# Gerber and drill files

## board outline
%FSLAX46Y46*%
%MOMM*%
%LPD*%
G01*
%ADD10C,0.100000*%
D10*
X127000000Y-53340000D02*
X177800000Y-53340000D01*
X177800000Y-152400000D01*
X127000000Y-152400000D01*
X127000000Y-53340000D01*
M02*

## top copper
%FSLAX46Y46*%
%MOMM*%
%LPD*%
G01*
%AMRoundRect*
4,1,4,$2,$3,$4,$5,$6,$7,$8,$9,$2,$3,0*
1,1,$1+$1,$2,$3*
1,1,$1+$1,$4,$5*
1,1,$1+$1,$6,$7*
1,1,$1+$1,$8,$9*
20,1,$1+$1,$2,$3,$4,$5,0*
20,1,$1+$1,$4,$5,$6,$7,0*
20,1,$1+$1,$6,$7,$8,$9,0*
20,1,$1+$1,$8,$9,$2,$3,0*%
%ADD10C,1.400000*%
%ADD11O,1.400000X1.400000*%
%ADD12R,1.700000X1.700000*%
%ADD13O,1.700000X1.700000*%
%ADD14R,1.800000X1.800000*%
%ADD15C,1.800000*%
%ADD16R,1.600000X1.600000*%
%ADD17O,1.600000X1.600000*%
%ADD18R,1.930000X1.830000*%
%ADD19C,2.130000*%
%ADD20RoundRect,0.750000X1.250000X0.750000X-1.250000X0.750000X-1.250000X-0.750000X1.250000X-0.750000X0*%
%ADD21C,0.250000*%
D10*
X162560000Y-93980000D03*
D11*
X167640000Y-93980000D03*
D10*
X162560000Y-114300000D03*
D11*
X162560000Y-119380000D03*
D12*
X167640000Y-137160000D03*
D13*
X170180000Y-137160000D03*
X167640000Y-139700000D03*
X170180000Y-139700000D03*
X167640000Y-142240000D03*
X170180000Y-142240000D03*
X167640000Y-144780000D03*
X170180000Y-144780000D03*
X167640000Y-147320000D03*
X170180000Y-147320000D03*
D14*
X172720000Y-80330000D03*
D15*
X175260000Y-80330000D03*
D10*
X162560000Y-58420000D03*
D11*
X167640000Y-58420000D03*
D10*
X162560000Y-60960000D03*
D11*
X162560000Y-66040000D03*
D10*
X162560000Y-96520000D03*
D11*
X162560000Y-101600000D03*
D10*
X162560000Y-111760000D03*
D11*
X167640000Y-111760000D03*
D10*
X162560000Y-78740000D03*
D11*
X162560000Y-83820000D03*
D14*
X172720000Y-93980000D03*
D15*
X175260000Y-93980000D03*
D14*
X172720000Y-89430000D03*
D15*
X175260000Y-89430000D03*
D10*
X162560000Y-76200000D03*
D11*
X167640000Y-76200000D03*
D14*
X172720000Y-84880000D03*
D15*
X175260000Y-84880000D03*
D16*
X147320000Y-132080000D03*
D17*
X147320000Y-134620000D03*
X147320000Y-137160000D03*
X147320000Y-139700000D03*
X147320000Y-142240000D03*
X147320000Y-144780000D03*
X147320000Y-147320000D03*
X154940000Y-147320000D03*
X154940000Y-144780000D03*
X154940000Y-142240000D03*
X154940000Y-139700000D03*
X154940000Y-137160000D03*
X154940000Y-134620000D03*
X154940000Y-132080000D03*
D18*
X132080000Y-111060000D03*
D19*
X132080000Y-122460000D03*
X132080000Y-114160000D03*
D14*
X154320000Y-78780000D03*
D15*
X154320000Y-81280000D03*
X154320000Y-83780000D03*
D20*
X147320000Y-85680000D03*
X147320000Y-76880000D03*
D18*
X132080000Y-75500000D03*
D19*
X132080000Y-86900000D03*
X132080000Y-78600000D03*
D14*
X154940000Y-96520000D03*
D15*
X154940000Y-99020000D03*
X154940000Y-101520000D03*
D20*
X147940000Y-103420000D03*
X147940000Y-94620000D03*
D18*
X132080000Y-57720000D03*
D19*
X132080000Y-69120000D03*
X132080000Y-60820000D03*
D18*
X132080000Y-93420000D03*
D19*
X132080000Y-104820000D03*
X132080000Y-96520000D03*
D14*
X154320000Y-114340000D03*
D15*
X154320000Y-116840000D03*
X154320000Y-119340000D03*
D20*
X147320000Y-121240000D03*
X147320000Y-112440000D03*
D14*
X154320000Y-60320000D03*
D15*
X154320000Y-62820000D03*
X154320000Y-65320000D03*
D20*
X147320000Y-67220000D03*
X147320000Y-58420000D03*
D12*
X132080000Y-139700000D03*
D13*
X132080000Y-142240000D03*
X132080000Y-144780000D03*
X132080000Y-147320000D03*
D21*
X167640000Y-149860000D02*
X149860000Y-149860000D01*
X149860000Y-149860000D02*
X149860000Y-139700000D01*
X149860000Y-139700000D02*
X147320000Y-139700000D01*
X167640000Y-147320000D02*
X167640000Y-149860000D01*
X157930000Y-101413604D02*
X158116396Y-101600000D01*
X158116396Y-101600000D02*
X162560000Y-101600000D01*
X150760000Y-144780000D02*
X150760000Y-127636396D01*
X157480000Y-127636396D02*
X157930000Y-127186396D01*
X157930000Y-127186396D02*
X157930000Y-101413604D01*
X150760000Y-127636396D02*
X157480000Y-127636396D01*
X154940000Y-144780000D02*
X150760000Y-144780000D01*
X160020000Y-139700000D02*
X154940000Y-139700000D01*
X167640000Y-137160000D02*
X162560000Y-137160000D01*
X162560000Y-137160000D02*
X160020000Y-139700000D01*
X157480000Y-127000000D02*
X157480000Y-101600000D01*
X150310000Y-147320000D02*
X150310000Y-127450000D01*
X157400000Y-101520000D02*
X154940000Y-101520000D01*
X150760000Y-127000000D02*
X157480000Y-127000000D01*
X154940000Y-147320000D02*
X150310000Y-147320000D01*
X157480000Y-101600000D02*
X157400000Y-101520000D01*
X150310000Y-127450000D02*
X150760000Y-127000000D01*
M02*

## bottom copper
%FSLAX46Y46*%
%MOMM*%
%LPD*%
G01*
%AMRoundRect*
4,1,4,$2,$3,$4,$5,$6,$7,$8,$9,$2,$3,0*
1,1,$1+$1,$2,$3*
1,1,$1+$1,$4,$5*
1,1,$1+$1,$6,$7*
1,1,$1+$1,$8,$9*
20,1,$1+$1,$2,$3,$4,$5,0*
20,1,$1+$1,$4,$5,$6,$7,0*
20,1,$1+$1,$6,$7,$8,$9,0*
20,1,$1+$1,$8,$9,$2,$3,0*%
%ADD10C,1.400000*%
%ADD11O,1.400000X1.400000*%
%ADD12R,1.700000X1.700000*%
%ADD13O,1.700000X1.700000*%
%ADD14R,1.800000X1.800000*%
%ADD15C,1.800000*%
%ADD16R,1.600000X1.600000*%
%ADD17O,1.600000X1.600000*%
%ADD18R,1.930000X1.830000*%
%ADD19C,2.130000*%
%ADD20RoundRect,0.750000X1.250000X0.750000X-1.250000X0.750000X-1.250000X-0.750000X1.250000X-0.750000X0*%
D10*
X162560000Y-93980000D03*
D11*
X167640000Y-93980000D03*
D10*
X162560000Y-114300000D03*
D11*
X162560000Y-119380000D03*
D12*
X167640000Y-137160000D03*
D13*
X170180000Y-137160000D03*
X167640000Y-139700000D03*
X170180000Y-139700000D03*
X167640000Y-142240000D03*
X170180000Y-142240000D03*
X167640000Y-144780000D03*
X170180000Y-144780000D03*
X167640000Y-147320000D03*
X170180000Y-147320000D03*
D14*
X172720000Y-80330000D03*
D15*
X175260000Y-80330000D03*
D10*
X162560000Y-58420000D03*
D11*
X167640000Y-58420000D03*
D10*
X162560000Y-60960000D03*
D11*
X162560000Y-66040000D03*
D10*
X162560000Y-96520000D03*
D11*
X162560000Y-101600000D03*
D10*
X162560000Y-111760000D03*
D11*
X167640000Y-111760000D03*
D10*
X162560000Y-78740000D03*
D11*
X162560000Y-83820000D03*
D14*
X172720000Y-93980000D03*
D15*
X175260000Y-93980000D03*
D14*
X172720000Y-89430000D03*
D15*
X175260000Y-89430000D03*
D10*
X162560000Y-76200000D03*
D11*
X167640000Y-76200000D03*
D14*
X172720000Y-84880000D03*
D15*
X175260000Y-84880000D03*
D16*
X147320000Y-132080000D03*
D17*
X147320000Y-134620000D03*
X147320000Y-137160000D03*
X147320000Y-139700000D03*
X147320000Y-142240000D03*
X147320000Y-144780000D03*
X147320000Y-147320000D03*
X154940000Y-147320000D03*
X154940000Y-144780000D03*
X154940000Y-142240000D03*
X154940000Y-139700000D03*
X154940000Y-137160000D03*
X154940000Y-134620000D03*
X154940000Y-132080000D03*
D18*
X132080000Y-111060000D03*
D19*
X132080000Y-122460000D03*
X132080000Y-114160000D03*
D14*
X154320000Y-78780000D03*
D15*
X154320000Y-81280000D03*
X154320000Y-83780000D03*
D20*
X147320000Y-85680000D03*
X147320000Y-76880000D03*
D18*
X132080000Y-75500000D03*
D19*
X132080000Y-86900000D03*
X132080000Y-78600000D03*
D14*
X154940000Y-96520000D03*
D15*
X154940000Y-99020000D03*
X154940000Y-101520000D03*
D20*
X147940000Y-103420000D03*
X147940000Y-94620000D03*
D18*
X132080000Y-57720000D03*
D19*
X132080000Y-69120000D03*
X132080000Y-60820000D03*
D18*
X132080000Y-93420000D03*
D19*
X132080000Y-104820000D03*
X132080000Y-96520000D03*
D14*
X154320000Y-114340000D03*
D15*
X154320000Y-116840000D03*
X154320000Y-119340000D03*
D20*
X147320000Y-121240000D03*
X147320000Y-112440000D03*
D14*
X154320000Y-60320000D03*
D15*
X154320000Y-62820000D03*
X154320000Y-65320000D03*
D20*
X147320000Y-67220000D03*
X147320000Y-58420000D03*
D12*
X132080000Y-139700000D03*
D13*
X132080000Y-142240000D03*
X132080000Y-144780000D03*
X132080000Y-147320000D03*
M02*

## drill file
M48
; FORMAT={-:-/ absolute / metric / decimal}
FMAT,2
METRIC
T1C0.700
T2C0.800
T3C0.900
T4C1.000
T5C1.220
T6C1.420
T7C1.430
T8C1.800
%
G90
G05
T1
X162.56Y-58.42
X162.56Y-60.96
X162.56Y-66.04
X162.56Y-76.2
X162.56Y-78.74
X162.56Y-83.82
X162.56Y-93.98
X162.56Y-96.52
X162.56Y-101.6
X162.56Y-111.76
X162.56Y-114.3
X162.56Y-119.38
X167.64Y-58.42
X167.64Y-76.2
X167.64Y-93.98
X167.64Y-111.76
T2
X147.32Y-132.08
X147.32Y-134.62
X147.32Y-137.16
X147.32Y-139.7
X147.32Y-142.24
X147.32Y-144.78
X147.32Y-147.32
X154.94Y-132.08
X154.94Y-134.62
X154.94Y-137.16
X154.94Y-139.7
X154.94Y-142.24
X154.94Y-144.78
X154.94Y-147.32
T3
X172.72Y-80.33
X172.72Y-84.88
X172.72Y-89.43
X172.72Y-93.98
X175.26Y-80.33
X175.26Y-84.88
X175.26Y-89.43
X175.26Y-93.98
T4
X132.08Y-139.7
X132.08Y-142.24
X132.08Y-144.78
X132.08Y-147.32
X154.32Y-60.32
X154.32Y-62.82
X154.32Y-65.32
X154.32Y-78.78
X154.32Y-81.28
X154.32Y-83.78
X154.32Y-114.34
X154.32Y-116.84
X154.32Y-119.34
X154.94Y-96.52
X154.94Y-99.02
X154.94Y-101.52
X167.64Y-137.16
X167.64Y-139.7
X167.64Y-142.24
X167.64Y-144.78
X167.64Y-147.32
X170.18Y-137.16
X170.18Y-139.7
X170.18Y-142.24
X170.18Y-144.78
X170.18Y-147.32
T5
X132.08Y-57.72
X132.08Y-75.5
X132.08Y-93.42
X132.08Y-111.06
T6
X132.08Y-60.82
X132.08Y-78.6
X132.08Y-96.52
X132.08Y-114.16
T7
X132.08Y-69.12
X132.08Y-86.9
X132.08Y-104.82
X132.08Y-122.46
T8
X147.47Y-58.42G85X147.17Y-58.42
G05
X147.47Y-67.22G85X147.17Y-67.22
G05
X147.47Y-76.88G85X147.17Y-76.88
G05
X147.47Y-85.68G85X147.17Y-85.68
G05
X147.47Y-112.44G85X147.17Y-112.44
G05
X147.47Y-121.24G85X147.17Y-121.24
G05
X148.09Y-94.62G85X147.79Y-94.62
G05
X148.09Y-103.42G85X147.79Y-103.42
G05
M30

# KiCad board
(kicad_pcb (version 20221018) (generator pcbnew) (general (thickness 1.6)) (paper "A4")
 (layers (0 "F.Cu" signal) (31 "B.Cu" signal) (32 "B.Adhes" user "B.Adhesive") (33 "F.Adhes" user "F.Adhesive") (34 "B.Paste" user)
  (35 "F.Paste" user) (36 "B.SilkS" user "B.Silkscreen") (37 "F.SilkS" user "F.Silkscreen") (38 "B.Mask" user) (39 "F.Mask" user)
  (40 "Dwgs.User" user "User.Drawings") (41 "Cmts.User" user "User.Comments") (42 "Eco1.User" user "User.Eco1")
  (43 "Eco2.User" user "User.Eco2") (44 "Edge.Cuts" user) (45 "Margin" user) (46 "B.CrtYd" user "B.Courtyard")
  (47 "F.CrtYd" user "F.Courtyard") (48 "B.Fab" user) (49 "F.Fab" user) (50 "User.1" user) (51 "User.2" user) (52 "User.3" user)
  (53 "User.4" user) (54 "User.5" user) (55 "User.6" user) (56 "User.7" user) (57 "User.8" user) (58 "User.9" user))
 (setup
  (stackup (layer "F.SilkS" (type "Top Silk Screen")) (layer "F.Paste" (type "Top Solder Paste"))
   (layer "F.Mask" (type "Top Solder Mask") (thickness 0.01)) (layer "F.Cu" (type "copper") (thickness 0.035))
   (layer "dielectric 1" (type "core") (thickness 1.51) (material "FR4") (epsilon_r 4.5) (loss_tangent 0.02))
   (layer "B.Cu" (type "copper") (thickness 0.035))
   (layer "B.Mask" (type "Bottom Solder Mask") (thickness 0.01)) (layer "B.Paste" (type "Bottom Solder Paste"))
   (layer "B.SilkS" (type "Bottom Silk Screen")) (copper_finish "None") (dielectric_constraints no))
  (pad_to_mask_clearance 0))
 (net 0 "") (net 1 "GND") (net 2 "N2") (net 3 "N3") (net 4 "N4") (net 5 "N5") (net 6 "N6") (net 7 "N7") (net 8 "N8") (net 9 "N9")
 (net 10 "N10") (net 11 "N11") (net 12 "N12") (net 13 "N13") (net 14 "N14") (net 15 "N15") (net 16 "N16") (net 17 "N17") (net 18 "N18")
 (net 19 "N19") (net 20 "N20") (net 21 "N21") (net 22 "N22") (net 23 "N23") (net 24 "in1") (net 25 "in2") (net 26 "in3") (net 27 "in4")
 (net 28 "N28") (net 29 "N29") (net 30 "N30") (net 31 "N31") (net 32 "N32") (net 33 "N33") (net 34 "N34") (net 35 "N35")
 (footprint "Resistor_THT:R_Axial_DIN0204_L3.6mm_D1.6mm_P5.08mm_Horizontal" (layer "F.Cu") (at 162.56 93.98)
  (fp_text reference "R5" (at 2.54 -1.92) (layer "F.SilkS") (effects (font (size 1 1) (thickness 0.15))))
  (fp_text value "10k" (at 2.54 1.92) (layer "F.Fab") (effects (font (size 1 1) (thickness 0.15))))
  (pad "1" thru_hole circle (at 0 0) (size 1.4 1.4) (drill 0.7) (layers "*.Cu" "*.Mask") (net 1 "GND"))
  (pad "2" thru_hole oval (at 5.08 0) (size 1.4 1.4) (drill 0.7) (layers "*.Cu" "*.Mask") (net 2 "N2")))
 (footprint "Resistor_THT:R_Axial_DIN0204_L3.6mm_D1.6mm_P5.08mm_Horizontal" (layer "F.Cu") (at 162.56 114.3 -90)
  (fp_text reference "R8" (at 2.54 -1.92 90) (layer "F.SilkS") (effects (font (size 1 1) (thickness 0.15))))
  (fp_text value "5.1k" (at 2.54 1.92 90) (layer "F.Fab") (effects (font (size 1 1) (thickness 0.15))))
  (pad "1" thru_hole circle (at 0 0 270) (size 1.4 1.4) (drill 0.7) (layers "*.Cu" "*.Mask") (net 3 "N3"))
  (pad "2" thru_hole oval (at 5.08 0 270) (size 1.4 1.4) (drill 0.7) (layers "*.Cu" "*.Mask") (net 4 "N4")))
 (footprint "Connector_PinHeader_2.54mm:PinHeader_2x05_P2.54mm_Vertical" (layer "F.Cu") (at 167.64 137.16)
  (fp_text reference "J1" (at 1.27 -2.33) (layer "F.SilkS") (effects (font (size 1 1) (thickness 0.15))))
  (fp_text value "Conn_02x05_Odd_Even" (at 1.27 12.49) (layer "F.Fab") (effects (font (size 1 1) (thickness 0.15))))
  (pad "1" thru_hole rect (at 0 0) (size 1.7 1.7) (drill 1) (layers "*.Cu" "*.Mask") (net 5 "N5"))
  (pad "2" thru_hole oval (at 2.54 0) (size 1.7 1.7) (drill 1) (layers "*.Cu" "*.Mask") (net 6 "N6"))
  (pad "3" thru_hole oval (at 0 2.54) (size 1.7 1.7) (drill 1) (layers "*.Cu" "*.Mask") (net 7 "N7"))
  (pad "4" thru_hole oval (at 2.54 2.54) (size 1.7 1.7) (drill 1) (layers "*.Cu" "*.Mask") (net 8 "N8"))
  (pad "5" thru_hole oval (at 0 5.08) (size 1.7 1.7) (drill 1) (layers "*.Cu" "*.Mask") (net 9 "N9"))
  (pad "6" thru_hole oval (at 2.54 5.08) (size 1.7 1.7) (drill 1) (layers "*.Cu" "*.Mask") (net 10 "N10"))
  (pad "7" thru_hole oval (at 0 7.62) (size 1.7 1.7) (drill 1) (layers "*.Cu" "*.Mask") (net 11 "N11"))
  (pad "8" thru_hole oval (at 2.54 7.62) (size 1.7 1.7) (drill 1) (layers "*.Cu" "*.Mask") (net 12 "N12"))
  (pad "9" thru_hole oval (at 0 10.16) (size 1.7 1.7) (drill 1) (layers "*.Cu" "*.Mask") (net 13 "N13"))
  (pad "10" thru_hole oval (at 2.54 10.16) (size 1.7 1.7) (drill 1) (layers "*.Cu" "*.Mask") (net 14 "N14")))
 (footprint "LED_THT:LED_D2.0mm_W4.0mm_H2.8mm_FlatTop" (layer "F.Cu") (at 172.72 80.33)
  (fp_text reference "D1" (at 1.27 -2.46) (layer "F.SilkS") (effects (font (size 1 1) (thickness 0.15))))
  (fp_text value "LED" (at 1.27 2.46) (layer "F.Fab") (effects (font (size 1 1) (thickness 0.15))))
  (pad "1" thru_hole rect (at 0 0) (size 1.8 1.8) (drill 0.9) (layers "*.Cu" "*.Mask") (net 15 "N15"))
  (pad "2" thru_hole circle (at 2.54 0) (size 1.8 1.8) (drill 0.9) (layers "*.Cu" "*.Mask") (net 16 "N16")))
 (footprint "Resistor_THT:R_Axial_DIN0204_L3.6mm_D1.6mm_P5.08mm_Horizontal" (layer "F.Cu") (at 162.56 58.42)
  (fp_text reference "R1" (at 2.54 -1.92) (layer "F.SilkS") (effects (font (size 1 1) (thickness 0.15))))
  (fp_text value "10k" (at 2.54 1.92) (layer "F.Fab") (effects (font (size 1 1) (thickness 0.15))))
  (pad "1" thru_hole circle (at 0 0) (size 1.4 1.4) (drill 0.7) (layers "*.Cu" "*.Mask") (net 1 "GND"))
  (pad "2" thru_hole oval (at 5.08 0) (size 1.4 1.4) (drill 0.7) (layers "*.Cu" "*.Mask") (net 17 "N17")))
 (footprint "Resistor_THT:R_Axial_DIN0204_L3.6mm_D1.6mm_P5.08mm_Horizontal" (layer "F.Cu") (at 162.56 60.96 -90)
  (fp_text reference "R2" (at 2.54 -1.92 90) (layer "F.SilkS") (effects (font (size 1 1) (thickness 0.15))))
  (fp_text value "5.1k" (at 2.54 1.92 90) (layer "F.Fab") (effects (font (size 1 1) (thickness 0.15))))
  (pad "1" thru_hole circle (at 0 0 270) (size 1.4 1.4) (drill 0.7) (layers "*.Cu" "*.Mask") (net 16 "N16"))
  (pad "2" thru_hole oval (at 5.08 0 270) (size 1.4 1.4) (drill 0.7) (layers "*.Cu" "*.Mask") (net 17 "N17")))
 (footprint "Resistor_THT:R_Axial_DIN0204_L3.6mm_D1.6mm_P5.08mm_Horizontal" (layer "F.Cu") (at 162.56 96.52 -90)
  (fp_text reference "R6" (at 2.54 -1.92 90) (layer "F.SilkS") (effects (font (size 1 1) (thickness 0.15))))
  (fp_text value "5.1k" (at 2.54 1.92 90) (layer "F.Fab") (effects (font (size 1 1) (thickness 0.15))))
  (pad "1" thru_hole circle (at 0 0 270) (size 1.4 1.4) (drill 0.7) (layers "*.Cu" "*.Mask") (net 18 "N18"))
  (pad "2" thru_hole oval (at 5.08 0 270) (size 1.4 1.4) (drill 0.7) (layers "*.Cu" "*.Mask") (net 2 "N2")))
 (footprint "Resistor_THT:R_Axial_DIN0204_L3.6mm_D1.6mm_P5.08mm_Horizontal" (layer "F.Cu") (at 162.56 111.76)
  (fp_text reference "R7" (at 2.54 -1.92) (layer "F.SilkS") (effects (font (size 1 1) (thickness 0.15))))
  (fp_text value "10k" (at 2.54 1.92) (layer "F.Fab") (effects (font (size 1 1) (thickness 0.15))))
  (pad "1" thru_hole circle (at 0 0) (size 1.4 1.4) (drill 0.7) (layers "*.Cu" "*.Mask") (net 1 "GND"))
  (pad "2" thru_hole oval (at 5.08 0) (size 1.4 1.4) (drill 0.7) (layers "*.Cu" "*.Mask") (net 4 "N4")))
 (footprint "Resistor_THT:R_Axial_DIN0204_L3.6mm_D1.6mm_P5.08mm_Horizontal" (layer "F.Cu") (at 162.56 78.74 -90)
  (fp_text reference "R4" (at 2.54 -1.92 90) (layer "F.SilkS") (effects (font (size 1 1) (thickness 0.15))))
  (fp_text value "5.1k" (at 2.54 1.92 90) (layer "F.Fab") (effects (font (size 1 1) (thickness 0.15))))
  (pad "1" thru_hole circle (at 0 0 270) (size 1.4 1.4) (drill 0.7) (layers "*.Cu" "*.Mask") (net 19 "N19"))
  (pad "2" thru_hole oval (at 5.08 0 270) (size 1.4 1.4) (drill 0.7) (layers "*.Cu" "*.Mask") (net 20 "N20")))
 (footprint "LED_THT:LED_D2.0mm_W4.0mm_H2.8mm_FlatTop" (layer "F.Cu") (at 172.72 93.98)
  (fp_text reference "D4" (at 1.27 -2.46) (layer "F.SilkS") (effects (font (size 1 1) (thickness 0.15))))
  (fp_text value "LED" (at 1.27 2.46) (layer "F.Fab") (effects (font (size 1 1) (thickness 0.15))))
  (pad "1" thru_hole rect (at 0 0) (size 1.8 1.8) (drill 0.9) (layers "*.Cu" "*.Mask") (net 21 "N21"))
  (pad "2" thru_hole circle (at 2.54 0) (size 1.8 1.8) (drill 0.9) (layers "*.Cu" "*.Mask") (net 3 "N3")))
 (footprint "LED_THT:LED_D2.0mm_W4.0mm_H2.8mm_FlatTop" (layer "F.Cu") (at 172.72 89.43)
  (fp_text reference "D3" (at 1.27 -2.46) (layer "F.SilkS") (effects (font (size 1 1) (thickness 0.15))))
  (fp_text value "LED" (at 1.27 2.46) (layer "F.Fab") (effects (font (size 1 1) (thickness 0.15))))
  (pad "1" thru_hole rect (at 0 0) (size 1.8 1.8) (drill 0.9) (layers "*.Cu" "*.Mask") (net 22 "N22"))
  (pad "2" thru_hole circle (at 2.54 0) (size 1.8 1.8) (drill 0.9) (layers "*.Cu" "*.Mask") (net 18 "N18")))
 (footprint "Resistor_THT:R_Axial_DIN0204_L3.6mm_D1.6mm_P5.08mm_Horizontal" (layer "F.Cu") (at 162.56 76.2)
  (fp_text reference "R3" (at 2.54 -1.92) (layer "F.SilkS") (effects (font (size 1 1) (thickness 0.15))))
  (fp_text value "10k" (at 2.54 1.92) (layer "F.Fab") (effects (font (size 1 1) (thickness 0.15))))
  (pad "1" thru_hole circle (at 0 0) (size 1.4 1.4) (drill 0.7) (layers "*.Cu" "*.Mask") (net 1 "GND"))
  (pad "2" thru_hole oval (at 5.08 0) (size 1.4 1.4) (drill 0.7) (layers "*.Cu" "*.Mask") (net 20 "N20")))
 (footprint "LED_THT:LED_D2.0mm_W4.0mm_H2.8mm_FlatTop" (layer "F.Cu") (at 172.72 84.88)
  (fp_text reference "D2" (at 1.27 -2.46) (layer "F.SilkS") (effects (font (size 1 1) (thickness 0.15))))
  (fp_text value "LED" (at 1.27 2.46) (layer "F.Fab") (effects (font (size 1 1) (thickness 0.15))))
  (pad "1" thru_hole rect (at 0 0) (size 1.8 1.8) (drill 0.9) (layers "*.Cu" "*.Mask") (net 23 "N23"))
  (pad "2" thru_hole circle (at 2.54 0) (size 1.8 1.8) (drill 0.9) (layers "*.Cu" "*.Mask") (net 19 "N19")))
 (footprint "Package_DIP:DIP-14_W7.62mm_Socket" (layer "F.Cu") (at 147.32 132.08)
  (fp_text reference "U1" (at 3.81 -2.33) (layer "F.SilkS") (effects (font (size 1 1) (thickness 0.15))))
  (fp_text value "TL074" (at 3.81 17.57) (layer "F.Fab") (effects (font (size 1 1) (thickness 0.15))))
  (pad "1" thru_hole rect (at 0 0) (size 1.6 1.6) (drill 0.8) (layers "*.Cu" "*.Mask") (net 16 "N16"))
  (pad "2" thru_hole oval (at 0 2.54) (size 1.6 1.6) (drill 0.8) (layers "*.Cu" "*.Mask") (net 17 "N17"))
  (pad "3" thru_hole oval (at 0 5.08) (size 1.6 1.6) (drill 0.8) (layers "*.Cu" "*.Mask") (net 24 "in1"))
  (pad "4" thru_hole oval (at 0 7.62) (size 1.6 1.6) (drill 0.8) (layers "*.Cu" "*.Mask") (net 13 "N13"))
  (pad "5" thru_hole oval (at 0 10.16) (size 1.6 1.6) (drill 0.8) (layers "*.Cu" "*.Mask") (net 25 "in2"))
  (pad "6" thru_hole oval (at 0 12.7) (size 1.6 1.6) (drill 0.8) (layers "*.Cu" "*.Mask") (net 20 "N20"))
  (pad "7" thru_hole oval (at 0 15.24) (size 1.6 1.6) (drill 0.8) (layers "*.Cu" "*.Mask") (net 19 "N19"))
  (pad "8" thru_hole oval (at 7.62 15.24) (size 1.6 1.6) (drill 0.8) (layers "*.Cu" "*.Mask") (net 18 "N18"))
  (pad "9" thru_hole oval (at 7.62 12.7) (size 1.6 1.6) (drill 0.8) (layers "*.Cu" "*.Mask") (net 2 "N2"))
  (pad "10" thru_hole oval (at 7.62 10.16) (size 1.6 1.6) (drill 0.8) (layers "*.Cu" "*.Mask") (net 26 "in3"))
  (pad "11" thru_hole oval (at 7.62 7.62) (size 1.6 1.6) (drill 0.8) (layers "*.Cu" "*.Mask") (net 5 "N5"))
  (pad "12" thru_hole oval (at 7.62 5.08) (size 1.6 1.6) (drill 0.8) (layers "*.Cu" "*.Mask") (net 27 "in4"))
  (pad "13" thru_hole oval (at 7.62 2.54) (size 1.6 1.6) (drill 0.8) (layers "*.Cu" "*.Mask") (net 4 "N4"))
  (pad "14" thru_hole oval (at 7.62 0) (size 1.6 1.6) (drill 0.8) (layers "*.Cu" "*.Mask") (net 3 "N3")))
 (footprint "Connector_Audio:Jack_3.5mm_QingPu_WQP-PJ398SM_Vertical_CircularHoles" (layer "B.Cu") (at 132.08 111.06 180)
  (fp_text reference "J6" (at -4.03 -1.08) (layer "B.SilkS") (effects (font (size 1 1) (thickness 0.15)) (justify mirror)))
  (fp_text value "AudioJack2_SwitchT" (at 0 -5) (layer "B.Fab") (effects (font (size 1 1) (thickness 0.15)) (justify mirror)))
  (pad "S" thru_hole rect (at 0 0) (size 1.93 1.83) (drill 1.22) (layers "*.Cu" "*.Mask") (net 1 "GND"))
  (pad "T" thru_hole circle (at 0 -11.4) (size 2.13 2.13) (drill 1.43) (layers "*.Cu" "*.Mask") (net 21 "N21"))
  (pad "TN" thru_hole circle (at 0 -3.1) (size 2.13 2.13) (drill 1.42) (layers "*.Cu" "*.Mask") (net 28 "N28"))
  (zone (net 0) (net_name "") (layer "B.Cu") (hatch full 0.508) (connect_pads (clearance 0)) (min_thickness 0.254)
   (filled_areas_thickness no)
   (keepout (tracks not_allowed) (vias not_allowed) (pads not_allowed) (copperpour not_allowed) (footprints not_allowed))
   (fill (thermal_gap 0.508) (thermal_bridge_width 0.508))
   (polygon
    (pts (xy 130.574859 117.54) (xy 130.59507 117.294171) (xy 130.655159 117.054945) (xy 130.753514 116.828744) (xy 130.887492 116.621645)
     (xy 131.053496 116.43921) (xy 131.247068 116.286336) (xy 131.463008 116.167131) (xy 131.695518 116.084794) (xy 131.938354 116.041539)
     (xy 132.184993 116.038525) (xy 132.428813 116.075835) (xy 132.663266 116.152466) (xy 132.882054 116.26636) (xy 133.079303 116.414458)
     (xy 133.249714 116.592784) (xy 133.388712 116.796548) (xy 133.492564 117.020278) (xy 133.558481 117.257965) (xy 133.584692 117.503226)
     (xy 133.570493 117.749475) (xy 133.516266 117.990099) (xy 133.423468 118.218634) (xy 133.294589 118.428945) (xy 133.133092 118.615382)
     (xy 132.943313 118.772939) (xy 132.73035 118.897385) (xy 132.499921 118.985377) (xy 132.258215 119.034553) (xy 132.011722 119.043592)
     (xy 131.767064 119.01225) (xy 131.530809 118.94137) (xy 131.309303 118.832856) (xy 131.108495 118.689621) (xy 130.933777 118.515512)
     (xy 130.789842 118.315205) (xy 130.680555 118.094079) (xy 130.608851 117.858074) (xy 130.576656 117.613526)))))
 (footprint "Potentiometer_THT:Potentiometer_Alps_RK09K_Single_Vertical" (layer "B.Cu") (at 154.32 78.78 180)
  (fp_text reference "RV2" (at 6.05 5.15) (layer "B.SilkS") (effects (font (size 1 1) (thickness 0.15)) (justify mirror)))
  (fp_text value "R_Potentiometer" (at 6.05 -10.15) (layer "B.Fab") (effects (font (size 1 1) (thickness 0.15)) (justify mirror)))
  (pad "1" thru_hole rect (at 0 0 180) (size 1.8 1.8) (drill 1) (layers "*.Cu" "*.Mask") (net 1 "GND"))
  (pad "2" thru_hole circle (at 0 -2.5 180) (size 1.8 1.8) (drill 1) (layers "*.Cu" "*.Mask") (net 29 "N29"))
  (pad "3" thru_hole circle (at 0 -5 180) (size 1.8 1.8) (drill 1) (layers "*.Cu" "*.Mask") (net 19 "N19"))
  (pad "MP" thru_hole roundrect (at 7 -6.9 180) (size 4 3) (drill oval 2.1 1.8) (layers "*.Cu" "*.Mask") (roundrect_rratio 0.25))
  (pad "MP" thru_hole roundrect (at 7 1.9 180) (size 4 3) (drill oval 2.1 1.8) (layers "*.Cu" "*.Mask") (roundrect_rratio 0.25)))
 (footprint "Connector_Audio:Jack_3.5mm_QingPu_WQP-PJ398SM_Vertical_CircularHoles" (layer "B.Cu") (at 132.08 75.5 180)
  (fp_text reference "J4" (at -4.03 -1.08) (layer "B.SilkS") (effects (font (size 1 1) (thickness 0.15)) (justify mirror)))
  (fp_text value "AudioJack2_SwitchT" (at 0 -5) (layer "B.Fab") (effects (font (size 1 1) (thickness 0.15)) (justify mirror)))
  (pad "S" thru_hole rect (at 0 0) (size 1.93 1.83) (drill 1.22) (layers "*.Cu" "*.Mask") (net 1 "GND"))
  (pad "T" thru_hole circle (at 0 -11.4) (size 2.13 2.13) (drill 1.43) (layers "*.Cu" "*.Mask") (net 23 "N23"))
  (pad "TN" thru_hole circle (at 0 -3.1) (size 2.13 2.13) (drill 1.42) (layers "*.Cu" "*.Mask") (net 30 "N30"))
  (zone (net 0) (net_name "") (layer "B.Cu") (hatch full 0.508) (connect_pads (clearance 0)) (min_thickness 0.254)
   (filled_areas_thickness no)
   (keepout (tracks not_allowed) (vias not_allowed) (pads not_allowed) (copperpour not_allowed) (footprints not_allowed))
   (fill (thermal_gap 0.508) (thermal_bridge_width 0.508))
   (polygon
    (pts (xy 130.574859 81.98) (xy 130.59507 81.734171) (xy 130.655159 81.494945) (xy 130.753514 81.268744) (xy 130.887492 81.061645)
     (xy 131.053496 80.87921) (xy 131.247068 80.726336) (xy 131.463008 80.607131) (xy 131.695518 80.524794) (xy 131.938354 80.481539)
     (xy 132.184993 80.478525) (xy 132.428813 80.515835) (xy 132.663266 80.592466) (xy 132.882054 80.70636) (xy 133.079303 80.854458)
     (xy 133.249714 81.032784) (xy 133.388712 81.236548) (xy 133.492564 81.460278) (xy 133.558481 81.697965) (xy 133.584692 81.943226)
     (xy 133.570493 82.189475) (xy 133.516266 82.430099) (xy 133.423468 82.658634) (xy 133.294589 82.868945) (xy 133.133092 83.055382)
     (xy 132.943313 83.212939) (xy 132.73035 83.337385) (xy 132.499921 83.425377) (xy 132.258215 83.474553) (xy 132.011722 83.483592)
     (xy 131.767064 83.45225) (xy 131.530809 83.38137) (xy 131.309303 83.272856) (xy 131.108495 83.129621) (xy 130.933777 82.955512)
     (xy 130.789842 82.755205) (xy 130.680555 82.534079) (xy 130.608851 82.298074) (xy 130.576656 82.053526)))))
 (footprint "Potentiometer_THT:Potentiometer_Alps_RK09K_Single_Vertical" (layer "B.Cu") (at 154.94 96.52 180)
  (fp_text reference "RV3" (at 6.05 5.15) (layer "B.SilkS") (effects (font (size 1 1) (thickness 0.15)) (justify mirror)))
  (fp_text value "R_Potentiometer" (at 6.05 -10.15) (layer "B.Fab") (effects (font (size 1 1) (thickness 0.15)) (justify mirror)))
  (pad "1" thru_hole rect (at 0 0 180) (size 1.8 1.8) (drill 1) (layers "*.Cu" "*.Mask") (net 1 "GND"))
  (pad "2" thru_hole circle (at 0 -2.5 180) (size 1.8 1.8) (drill 1) (layers "*.Cu" "*.Mask") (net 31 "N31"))
  (pad "3" thru_hole circle (at 0 -5 180) (size 1.8 1.8) (drill 1) (layers "*.Cu" "*.Mask") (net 18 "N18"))
  (pad "MP" thru_hole roundrect (at 7 -6.9 180) (size 4 3) (drill oval 2.1 1.8) (layers "*.Cu" "*.Mask") (roundrect_rratio 0.25))
  (pad "MP" thru_hole roundrect (at 7 1.9 180) (size 4 3) (drill oval 2.1 1.8) (layers "*.Cu" "*.Mask") (roundrect_rratio 0.25)))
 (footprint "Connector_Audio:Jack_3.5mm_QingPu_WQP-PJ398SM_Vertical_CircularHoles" (layer "B.Cu") (at 132.08 57.72 180)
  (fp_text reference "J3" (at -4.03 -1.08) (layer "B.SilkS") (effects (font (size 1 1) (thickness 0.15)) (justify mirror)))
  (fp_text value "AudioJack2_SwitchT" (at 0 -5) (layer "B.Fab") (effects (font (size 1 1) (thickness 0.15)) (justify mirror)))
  (pad "S" thru_hole rect (at 0 0) (size 1.93 1.83) (drill 1.22) (layers "*.Cu" "*.Mask") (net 1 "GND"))
  (pad "T" thru_hole circle (at 0 -11.4) (size 2.13 2.13) (drill 1.43) (layers "*.Cu" "*.Mask") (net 15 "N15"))
  (pad "TN" thru_hole circle (at 0 -3.1) (size 2.13 2.13) (drill 1.42) (layers "*.Cu" "*.Mask") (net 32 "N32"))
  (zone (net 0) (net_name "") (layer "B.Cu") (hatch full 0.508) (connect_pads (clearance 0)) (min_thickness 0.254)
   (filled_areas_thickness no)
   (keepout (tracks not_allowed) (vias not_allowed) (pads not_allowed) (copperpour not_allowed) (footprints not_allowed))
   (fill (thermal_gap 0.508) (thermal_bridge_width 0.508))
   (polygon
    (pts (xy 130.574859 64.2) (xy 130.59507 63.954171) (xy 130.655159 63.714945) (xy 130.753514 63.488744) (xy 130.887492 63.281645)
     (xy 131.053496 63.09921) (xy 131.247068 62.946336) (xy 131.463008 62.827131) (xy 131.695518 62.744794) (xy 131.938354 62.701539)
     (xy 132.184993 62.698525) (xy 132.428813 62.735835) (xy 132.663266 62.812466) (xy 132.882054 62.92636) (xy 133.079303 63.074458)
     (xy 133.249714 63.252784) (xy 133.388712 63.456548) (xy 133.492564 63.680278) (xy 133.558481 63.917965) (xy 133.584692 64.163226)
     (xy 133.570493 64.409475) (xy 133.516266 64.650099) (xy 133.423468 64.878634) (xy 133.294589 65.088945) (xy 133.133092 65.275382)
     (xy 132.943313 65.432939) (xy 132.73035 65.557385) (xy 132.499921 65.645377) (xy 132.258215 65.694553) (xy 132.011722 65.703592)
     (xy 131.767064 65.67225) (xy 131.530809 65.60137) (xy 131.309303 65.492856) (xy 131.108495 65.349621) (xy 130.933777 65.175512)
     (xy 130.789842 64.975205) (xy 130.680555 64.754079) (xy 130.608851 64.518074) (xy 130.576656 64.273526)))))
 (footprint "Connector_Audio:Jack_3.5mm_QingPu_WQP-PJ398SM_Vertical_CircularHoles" (layer "B.Cu") (at 132.08 93.42 180)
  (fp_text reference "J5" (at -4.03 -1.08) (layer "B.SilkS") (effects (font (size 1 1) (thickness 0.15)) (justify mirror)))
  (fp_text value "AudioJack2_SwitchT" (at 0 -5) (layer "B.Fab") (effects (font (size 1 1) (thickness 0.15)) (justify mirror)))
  (pad "S" thru_hole rect (at 0 0) (size 1.93 1.83) (drill 1.22) (layers "*.Cu" "*.Mask") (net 1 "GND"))
  (pad "T" thru_hole circle (at 0 -11.4) (size 2.13 2.13) (drill 1.43) (layers "*.Cu" "*.Mask") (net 22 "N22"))
  (pad "TN" thru_hole circle (at 0 -3.1) (size 2.13 2.13) (drill 1.42) (layers "*.Cu" "*.Mask") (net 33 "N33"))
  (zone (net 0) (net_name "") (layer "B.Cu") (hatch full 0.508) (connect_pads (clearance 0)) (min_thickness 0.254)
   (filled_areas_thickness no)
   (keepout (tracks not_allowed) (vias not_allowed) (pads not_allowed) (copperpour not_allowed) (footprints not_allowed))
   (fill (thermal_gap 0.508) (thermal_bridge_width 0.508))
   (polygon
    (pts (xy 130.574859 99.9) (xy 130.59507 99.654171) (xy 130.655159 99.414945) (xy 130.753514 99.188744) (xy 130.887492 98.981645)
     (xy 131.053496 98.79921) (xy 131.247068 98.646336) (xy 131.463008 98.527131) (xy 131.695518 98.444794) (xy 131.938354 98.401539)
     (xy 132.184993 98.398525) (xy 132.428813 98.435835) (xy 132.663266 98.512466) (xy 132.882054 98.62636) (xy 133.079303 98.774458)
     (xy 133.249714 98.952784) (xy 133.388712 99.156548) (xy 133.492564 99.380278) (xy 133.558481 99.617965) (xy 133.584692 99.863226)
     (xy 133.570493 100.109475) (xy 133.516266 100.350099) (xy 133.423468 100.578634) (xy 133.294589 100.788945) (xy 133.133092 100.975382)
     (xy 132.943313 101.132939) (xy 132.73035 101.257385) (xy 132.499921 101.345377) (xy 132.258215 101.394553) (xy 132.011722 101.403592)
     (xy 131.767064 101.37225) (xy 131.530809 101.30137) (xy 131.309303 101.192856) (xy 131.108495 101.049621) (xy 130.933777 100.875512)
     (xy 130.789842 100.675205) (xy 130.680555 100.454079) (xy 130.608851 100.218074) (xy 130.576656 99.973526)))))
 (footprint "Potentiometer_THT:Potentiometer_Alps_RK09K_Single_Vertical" (layer "B.Cu") (at 154.32 114.34 180)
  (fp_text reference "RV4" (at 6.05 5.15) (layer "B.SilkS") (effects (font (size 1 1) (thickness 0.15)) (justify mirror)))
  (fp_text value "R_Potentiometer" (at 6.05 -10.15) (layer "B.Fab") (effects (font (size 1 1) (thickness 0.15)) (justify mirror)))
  (pad "1" thru_hole rect (at 0 0 180) (size 1.8 1.8) (drill 1) (layers "*.Cu" "*.Mask") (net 1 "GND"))
  (pad "2" thru_hole circle (at 0 -2.5 180) (size 1.8 1.8) (drill 1) (layers "*.Cu" "*.Mask") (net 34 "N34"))
  (pad "3" thru_hole circle (at 0 -5 180) (size 1.8 1.8) (drill 1) (layers "*.Cu" "*.Mask") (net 3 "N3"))
  (pad "MP" thru_hole roundrect (at 7 -6.9 180) (size 4 3) (drill oval 2.1 1.8) (layers "*.Cu" "*.Mask") (roundrect_rratio 0.25))
  (pad "MP" thru_hole roundrect (at 7 1.9 180) (size 4 3) (drill oval 2.1 1.8) (layers "*.Cu" "*.Mask") (roundrect_rratio 0.25)))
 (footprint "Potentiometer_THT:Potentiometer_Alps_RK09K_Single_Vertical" (layer "B.Cu") (at 154.32 60.32 180)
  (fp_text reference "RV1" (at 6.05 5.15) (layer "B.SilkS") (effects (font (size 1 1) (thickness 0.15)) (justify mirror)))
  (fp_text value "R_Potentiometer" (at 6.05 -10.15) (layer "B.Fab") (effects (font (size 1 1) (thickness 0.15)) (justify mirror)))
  (pad "1" thru_hole rect (at 0 0 180) (size 1.8 1.8) (drill 1) (layers "*.Cu" "*.Mask") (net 1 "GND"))
  (pad "2" thru_hole circle (at 0 -2.5 180) (size 1.8 1.8) (drill 1) (layers "*.Cu" "*.Mask") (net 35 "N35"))
  (pad "3" thru_hole circle (at 0 -5 180) (size 1.8 1.8) (drill 1) (layers "*.Cu" "*.Mask") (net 16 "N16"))
  (pad "MP" thru_hole roundrect (at 7 -6.9 180) (size 4 3) (drill oval 2.1 1.8) (layers "*.Cu" "*.Mask") (roundrect_rratio 0.25))
  (pad "MP" thru_hole roundrect (at 7 1.9 180) (size 4 3) (drill oval 2.1 1.8) (layers "*.Cu" "*.Mask") (roundrect_rratio 0.25)))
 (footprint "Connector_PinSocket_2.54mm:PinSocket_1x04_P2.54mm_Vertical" (layer "B.Cu") (at 132.08 139.7 180)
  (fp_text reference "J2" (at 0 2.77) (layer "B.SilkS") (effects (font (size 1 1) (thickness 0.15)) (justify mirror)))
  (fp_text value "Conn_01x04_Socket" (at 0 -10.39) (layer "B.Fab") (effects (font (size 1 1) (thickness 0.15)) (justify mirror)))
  (pad "1" thru_hole rect (at 0 0 180) (size 1.7 1.7) (drill 1) (layers "*.Cu" "*.Mask") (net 24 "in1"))
  (pad "2" thru_hole oval (at 0 -2.54 180) (size 1.7 1.7) (drill 1) (layers "*.Cu" "*.Mask") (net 25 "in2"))
  (pad "3" thru_hole oval (at 0 -5.08 180) (size 1.7 1.7) (drill 1) (layers "*.Cu" "*.Mask") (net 26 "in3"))
  (pad "4" thru_hole oval (at 0 -7.62 180) (size 1.7 1.7) (drill 1) (layers "*.Cu" "*.Mask") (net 27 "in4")))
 (gr_rect (start 127 53.34) (end 177.8 152.4) (stroke (width 0.1) (type default)) (fill none) (layer "Edge.Cuts"))
 (segment (start 167.64 149.86) (end 149.86 149.86) (width 0.25) (layer "F.Cu") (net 13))
 (segment (start 149.86 149.86) (end 149.86 139.7) (width 0.25) (layer "F.Cu") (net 13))
 (segment (start 149.86 139.7) (end 147.32 139.7) (width 0.25) (layer "F.Cu") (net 13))
 (segment (start 167.64 147.32) (end 167.64 149.86) (width 0.25) (layer "F.Cu") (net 13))
 (segment (start 157.93 101.413604) (end 158.116396 101.6) (width 0.25) (layer "F.Cu") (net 2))
 (segment (start 158.116396 101.6) (end 162.56 101.6) (width 0.25) (layer "F.Cu") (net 2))
 (segment (start 150.76 144.78) (end 150.76 127.636396) (width 0.25) (layer "F.Cu") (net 2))
 (segment (start 157.48 127.636396) (end 157.93 127.186396) (width 0.25) (layer "F.Cu") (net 2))
 (segment (start 157.93 127.186396) (end 157.93 101.413604) (width 0.25) (layer "F.Cu") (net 2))
 (segment (start 150.76 127.636396) (end 157.48 127.636396) (width 0.25) (layer "F.Cu") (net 2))
 (segment (start 154.94 144.78) (end 150.76 144.78) (width 0.25) (layer "F.Cu") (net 2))
 (segment (start 160.02 139.7) (end 154.94 139.7) (width 0.25) (layer "F.Cu") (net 5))
 (segment (start 167.64 137.16) (end 162.56 137.16) (width 0.25) (layer "F.Cu") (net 5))
 (segment (start 162.56 137.16) (end 160.02 139.7) (width 0.25) (layer "F.Cu") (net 5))
 (segment (start 157.48 127) (end 157.48 101.6) (width 0.25) (layer "F.Cu") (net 18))
 (segment (start 150.31 147.32) (end 150.31 127.45) (width 0.25) (layer "F.Cu") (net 18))
 (segment (start 157.4 101.52) (end 154.94 101.52) (width 0.25) (layer "F.Cu") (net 18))
 (segment (start 150.76 127) (end 157.48 127) (width 0.25) (layer "F.Cu") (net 18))
 (segment (start 154.94 147.32) (end 150.31 147.32) (width 0.25) (layer "F.Cu") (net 18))
 (segment (start 157.48 101.6) (end 157.4 101.52) (width 0.25) (layer "F.Cu") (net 18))
 (segment (start 150.31 127.45) (end 150.76 127) (width 0.25) (layer "F.Cu") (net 18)))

